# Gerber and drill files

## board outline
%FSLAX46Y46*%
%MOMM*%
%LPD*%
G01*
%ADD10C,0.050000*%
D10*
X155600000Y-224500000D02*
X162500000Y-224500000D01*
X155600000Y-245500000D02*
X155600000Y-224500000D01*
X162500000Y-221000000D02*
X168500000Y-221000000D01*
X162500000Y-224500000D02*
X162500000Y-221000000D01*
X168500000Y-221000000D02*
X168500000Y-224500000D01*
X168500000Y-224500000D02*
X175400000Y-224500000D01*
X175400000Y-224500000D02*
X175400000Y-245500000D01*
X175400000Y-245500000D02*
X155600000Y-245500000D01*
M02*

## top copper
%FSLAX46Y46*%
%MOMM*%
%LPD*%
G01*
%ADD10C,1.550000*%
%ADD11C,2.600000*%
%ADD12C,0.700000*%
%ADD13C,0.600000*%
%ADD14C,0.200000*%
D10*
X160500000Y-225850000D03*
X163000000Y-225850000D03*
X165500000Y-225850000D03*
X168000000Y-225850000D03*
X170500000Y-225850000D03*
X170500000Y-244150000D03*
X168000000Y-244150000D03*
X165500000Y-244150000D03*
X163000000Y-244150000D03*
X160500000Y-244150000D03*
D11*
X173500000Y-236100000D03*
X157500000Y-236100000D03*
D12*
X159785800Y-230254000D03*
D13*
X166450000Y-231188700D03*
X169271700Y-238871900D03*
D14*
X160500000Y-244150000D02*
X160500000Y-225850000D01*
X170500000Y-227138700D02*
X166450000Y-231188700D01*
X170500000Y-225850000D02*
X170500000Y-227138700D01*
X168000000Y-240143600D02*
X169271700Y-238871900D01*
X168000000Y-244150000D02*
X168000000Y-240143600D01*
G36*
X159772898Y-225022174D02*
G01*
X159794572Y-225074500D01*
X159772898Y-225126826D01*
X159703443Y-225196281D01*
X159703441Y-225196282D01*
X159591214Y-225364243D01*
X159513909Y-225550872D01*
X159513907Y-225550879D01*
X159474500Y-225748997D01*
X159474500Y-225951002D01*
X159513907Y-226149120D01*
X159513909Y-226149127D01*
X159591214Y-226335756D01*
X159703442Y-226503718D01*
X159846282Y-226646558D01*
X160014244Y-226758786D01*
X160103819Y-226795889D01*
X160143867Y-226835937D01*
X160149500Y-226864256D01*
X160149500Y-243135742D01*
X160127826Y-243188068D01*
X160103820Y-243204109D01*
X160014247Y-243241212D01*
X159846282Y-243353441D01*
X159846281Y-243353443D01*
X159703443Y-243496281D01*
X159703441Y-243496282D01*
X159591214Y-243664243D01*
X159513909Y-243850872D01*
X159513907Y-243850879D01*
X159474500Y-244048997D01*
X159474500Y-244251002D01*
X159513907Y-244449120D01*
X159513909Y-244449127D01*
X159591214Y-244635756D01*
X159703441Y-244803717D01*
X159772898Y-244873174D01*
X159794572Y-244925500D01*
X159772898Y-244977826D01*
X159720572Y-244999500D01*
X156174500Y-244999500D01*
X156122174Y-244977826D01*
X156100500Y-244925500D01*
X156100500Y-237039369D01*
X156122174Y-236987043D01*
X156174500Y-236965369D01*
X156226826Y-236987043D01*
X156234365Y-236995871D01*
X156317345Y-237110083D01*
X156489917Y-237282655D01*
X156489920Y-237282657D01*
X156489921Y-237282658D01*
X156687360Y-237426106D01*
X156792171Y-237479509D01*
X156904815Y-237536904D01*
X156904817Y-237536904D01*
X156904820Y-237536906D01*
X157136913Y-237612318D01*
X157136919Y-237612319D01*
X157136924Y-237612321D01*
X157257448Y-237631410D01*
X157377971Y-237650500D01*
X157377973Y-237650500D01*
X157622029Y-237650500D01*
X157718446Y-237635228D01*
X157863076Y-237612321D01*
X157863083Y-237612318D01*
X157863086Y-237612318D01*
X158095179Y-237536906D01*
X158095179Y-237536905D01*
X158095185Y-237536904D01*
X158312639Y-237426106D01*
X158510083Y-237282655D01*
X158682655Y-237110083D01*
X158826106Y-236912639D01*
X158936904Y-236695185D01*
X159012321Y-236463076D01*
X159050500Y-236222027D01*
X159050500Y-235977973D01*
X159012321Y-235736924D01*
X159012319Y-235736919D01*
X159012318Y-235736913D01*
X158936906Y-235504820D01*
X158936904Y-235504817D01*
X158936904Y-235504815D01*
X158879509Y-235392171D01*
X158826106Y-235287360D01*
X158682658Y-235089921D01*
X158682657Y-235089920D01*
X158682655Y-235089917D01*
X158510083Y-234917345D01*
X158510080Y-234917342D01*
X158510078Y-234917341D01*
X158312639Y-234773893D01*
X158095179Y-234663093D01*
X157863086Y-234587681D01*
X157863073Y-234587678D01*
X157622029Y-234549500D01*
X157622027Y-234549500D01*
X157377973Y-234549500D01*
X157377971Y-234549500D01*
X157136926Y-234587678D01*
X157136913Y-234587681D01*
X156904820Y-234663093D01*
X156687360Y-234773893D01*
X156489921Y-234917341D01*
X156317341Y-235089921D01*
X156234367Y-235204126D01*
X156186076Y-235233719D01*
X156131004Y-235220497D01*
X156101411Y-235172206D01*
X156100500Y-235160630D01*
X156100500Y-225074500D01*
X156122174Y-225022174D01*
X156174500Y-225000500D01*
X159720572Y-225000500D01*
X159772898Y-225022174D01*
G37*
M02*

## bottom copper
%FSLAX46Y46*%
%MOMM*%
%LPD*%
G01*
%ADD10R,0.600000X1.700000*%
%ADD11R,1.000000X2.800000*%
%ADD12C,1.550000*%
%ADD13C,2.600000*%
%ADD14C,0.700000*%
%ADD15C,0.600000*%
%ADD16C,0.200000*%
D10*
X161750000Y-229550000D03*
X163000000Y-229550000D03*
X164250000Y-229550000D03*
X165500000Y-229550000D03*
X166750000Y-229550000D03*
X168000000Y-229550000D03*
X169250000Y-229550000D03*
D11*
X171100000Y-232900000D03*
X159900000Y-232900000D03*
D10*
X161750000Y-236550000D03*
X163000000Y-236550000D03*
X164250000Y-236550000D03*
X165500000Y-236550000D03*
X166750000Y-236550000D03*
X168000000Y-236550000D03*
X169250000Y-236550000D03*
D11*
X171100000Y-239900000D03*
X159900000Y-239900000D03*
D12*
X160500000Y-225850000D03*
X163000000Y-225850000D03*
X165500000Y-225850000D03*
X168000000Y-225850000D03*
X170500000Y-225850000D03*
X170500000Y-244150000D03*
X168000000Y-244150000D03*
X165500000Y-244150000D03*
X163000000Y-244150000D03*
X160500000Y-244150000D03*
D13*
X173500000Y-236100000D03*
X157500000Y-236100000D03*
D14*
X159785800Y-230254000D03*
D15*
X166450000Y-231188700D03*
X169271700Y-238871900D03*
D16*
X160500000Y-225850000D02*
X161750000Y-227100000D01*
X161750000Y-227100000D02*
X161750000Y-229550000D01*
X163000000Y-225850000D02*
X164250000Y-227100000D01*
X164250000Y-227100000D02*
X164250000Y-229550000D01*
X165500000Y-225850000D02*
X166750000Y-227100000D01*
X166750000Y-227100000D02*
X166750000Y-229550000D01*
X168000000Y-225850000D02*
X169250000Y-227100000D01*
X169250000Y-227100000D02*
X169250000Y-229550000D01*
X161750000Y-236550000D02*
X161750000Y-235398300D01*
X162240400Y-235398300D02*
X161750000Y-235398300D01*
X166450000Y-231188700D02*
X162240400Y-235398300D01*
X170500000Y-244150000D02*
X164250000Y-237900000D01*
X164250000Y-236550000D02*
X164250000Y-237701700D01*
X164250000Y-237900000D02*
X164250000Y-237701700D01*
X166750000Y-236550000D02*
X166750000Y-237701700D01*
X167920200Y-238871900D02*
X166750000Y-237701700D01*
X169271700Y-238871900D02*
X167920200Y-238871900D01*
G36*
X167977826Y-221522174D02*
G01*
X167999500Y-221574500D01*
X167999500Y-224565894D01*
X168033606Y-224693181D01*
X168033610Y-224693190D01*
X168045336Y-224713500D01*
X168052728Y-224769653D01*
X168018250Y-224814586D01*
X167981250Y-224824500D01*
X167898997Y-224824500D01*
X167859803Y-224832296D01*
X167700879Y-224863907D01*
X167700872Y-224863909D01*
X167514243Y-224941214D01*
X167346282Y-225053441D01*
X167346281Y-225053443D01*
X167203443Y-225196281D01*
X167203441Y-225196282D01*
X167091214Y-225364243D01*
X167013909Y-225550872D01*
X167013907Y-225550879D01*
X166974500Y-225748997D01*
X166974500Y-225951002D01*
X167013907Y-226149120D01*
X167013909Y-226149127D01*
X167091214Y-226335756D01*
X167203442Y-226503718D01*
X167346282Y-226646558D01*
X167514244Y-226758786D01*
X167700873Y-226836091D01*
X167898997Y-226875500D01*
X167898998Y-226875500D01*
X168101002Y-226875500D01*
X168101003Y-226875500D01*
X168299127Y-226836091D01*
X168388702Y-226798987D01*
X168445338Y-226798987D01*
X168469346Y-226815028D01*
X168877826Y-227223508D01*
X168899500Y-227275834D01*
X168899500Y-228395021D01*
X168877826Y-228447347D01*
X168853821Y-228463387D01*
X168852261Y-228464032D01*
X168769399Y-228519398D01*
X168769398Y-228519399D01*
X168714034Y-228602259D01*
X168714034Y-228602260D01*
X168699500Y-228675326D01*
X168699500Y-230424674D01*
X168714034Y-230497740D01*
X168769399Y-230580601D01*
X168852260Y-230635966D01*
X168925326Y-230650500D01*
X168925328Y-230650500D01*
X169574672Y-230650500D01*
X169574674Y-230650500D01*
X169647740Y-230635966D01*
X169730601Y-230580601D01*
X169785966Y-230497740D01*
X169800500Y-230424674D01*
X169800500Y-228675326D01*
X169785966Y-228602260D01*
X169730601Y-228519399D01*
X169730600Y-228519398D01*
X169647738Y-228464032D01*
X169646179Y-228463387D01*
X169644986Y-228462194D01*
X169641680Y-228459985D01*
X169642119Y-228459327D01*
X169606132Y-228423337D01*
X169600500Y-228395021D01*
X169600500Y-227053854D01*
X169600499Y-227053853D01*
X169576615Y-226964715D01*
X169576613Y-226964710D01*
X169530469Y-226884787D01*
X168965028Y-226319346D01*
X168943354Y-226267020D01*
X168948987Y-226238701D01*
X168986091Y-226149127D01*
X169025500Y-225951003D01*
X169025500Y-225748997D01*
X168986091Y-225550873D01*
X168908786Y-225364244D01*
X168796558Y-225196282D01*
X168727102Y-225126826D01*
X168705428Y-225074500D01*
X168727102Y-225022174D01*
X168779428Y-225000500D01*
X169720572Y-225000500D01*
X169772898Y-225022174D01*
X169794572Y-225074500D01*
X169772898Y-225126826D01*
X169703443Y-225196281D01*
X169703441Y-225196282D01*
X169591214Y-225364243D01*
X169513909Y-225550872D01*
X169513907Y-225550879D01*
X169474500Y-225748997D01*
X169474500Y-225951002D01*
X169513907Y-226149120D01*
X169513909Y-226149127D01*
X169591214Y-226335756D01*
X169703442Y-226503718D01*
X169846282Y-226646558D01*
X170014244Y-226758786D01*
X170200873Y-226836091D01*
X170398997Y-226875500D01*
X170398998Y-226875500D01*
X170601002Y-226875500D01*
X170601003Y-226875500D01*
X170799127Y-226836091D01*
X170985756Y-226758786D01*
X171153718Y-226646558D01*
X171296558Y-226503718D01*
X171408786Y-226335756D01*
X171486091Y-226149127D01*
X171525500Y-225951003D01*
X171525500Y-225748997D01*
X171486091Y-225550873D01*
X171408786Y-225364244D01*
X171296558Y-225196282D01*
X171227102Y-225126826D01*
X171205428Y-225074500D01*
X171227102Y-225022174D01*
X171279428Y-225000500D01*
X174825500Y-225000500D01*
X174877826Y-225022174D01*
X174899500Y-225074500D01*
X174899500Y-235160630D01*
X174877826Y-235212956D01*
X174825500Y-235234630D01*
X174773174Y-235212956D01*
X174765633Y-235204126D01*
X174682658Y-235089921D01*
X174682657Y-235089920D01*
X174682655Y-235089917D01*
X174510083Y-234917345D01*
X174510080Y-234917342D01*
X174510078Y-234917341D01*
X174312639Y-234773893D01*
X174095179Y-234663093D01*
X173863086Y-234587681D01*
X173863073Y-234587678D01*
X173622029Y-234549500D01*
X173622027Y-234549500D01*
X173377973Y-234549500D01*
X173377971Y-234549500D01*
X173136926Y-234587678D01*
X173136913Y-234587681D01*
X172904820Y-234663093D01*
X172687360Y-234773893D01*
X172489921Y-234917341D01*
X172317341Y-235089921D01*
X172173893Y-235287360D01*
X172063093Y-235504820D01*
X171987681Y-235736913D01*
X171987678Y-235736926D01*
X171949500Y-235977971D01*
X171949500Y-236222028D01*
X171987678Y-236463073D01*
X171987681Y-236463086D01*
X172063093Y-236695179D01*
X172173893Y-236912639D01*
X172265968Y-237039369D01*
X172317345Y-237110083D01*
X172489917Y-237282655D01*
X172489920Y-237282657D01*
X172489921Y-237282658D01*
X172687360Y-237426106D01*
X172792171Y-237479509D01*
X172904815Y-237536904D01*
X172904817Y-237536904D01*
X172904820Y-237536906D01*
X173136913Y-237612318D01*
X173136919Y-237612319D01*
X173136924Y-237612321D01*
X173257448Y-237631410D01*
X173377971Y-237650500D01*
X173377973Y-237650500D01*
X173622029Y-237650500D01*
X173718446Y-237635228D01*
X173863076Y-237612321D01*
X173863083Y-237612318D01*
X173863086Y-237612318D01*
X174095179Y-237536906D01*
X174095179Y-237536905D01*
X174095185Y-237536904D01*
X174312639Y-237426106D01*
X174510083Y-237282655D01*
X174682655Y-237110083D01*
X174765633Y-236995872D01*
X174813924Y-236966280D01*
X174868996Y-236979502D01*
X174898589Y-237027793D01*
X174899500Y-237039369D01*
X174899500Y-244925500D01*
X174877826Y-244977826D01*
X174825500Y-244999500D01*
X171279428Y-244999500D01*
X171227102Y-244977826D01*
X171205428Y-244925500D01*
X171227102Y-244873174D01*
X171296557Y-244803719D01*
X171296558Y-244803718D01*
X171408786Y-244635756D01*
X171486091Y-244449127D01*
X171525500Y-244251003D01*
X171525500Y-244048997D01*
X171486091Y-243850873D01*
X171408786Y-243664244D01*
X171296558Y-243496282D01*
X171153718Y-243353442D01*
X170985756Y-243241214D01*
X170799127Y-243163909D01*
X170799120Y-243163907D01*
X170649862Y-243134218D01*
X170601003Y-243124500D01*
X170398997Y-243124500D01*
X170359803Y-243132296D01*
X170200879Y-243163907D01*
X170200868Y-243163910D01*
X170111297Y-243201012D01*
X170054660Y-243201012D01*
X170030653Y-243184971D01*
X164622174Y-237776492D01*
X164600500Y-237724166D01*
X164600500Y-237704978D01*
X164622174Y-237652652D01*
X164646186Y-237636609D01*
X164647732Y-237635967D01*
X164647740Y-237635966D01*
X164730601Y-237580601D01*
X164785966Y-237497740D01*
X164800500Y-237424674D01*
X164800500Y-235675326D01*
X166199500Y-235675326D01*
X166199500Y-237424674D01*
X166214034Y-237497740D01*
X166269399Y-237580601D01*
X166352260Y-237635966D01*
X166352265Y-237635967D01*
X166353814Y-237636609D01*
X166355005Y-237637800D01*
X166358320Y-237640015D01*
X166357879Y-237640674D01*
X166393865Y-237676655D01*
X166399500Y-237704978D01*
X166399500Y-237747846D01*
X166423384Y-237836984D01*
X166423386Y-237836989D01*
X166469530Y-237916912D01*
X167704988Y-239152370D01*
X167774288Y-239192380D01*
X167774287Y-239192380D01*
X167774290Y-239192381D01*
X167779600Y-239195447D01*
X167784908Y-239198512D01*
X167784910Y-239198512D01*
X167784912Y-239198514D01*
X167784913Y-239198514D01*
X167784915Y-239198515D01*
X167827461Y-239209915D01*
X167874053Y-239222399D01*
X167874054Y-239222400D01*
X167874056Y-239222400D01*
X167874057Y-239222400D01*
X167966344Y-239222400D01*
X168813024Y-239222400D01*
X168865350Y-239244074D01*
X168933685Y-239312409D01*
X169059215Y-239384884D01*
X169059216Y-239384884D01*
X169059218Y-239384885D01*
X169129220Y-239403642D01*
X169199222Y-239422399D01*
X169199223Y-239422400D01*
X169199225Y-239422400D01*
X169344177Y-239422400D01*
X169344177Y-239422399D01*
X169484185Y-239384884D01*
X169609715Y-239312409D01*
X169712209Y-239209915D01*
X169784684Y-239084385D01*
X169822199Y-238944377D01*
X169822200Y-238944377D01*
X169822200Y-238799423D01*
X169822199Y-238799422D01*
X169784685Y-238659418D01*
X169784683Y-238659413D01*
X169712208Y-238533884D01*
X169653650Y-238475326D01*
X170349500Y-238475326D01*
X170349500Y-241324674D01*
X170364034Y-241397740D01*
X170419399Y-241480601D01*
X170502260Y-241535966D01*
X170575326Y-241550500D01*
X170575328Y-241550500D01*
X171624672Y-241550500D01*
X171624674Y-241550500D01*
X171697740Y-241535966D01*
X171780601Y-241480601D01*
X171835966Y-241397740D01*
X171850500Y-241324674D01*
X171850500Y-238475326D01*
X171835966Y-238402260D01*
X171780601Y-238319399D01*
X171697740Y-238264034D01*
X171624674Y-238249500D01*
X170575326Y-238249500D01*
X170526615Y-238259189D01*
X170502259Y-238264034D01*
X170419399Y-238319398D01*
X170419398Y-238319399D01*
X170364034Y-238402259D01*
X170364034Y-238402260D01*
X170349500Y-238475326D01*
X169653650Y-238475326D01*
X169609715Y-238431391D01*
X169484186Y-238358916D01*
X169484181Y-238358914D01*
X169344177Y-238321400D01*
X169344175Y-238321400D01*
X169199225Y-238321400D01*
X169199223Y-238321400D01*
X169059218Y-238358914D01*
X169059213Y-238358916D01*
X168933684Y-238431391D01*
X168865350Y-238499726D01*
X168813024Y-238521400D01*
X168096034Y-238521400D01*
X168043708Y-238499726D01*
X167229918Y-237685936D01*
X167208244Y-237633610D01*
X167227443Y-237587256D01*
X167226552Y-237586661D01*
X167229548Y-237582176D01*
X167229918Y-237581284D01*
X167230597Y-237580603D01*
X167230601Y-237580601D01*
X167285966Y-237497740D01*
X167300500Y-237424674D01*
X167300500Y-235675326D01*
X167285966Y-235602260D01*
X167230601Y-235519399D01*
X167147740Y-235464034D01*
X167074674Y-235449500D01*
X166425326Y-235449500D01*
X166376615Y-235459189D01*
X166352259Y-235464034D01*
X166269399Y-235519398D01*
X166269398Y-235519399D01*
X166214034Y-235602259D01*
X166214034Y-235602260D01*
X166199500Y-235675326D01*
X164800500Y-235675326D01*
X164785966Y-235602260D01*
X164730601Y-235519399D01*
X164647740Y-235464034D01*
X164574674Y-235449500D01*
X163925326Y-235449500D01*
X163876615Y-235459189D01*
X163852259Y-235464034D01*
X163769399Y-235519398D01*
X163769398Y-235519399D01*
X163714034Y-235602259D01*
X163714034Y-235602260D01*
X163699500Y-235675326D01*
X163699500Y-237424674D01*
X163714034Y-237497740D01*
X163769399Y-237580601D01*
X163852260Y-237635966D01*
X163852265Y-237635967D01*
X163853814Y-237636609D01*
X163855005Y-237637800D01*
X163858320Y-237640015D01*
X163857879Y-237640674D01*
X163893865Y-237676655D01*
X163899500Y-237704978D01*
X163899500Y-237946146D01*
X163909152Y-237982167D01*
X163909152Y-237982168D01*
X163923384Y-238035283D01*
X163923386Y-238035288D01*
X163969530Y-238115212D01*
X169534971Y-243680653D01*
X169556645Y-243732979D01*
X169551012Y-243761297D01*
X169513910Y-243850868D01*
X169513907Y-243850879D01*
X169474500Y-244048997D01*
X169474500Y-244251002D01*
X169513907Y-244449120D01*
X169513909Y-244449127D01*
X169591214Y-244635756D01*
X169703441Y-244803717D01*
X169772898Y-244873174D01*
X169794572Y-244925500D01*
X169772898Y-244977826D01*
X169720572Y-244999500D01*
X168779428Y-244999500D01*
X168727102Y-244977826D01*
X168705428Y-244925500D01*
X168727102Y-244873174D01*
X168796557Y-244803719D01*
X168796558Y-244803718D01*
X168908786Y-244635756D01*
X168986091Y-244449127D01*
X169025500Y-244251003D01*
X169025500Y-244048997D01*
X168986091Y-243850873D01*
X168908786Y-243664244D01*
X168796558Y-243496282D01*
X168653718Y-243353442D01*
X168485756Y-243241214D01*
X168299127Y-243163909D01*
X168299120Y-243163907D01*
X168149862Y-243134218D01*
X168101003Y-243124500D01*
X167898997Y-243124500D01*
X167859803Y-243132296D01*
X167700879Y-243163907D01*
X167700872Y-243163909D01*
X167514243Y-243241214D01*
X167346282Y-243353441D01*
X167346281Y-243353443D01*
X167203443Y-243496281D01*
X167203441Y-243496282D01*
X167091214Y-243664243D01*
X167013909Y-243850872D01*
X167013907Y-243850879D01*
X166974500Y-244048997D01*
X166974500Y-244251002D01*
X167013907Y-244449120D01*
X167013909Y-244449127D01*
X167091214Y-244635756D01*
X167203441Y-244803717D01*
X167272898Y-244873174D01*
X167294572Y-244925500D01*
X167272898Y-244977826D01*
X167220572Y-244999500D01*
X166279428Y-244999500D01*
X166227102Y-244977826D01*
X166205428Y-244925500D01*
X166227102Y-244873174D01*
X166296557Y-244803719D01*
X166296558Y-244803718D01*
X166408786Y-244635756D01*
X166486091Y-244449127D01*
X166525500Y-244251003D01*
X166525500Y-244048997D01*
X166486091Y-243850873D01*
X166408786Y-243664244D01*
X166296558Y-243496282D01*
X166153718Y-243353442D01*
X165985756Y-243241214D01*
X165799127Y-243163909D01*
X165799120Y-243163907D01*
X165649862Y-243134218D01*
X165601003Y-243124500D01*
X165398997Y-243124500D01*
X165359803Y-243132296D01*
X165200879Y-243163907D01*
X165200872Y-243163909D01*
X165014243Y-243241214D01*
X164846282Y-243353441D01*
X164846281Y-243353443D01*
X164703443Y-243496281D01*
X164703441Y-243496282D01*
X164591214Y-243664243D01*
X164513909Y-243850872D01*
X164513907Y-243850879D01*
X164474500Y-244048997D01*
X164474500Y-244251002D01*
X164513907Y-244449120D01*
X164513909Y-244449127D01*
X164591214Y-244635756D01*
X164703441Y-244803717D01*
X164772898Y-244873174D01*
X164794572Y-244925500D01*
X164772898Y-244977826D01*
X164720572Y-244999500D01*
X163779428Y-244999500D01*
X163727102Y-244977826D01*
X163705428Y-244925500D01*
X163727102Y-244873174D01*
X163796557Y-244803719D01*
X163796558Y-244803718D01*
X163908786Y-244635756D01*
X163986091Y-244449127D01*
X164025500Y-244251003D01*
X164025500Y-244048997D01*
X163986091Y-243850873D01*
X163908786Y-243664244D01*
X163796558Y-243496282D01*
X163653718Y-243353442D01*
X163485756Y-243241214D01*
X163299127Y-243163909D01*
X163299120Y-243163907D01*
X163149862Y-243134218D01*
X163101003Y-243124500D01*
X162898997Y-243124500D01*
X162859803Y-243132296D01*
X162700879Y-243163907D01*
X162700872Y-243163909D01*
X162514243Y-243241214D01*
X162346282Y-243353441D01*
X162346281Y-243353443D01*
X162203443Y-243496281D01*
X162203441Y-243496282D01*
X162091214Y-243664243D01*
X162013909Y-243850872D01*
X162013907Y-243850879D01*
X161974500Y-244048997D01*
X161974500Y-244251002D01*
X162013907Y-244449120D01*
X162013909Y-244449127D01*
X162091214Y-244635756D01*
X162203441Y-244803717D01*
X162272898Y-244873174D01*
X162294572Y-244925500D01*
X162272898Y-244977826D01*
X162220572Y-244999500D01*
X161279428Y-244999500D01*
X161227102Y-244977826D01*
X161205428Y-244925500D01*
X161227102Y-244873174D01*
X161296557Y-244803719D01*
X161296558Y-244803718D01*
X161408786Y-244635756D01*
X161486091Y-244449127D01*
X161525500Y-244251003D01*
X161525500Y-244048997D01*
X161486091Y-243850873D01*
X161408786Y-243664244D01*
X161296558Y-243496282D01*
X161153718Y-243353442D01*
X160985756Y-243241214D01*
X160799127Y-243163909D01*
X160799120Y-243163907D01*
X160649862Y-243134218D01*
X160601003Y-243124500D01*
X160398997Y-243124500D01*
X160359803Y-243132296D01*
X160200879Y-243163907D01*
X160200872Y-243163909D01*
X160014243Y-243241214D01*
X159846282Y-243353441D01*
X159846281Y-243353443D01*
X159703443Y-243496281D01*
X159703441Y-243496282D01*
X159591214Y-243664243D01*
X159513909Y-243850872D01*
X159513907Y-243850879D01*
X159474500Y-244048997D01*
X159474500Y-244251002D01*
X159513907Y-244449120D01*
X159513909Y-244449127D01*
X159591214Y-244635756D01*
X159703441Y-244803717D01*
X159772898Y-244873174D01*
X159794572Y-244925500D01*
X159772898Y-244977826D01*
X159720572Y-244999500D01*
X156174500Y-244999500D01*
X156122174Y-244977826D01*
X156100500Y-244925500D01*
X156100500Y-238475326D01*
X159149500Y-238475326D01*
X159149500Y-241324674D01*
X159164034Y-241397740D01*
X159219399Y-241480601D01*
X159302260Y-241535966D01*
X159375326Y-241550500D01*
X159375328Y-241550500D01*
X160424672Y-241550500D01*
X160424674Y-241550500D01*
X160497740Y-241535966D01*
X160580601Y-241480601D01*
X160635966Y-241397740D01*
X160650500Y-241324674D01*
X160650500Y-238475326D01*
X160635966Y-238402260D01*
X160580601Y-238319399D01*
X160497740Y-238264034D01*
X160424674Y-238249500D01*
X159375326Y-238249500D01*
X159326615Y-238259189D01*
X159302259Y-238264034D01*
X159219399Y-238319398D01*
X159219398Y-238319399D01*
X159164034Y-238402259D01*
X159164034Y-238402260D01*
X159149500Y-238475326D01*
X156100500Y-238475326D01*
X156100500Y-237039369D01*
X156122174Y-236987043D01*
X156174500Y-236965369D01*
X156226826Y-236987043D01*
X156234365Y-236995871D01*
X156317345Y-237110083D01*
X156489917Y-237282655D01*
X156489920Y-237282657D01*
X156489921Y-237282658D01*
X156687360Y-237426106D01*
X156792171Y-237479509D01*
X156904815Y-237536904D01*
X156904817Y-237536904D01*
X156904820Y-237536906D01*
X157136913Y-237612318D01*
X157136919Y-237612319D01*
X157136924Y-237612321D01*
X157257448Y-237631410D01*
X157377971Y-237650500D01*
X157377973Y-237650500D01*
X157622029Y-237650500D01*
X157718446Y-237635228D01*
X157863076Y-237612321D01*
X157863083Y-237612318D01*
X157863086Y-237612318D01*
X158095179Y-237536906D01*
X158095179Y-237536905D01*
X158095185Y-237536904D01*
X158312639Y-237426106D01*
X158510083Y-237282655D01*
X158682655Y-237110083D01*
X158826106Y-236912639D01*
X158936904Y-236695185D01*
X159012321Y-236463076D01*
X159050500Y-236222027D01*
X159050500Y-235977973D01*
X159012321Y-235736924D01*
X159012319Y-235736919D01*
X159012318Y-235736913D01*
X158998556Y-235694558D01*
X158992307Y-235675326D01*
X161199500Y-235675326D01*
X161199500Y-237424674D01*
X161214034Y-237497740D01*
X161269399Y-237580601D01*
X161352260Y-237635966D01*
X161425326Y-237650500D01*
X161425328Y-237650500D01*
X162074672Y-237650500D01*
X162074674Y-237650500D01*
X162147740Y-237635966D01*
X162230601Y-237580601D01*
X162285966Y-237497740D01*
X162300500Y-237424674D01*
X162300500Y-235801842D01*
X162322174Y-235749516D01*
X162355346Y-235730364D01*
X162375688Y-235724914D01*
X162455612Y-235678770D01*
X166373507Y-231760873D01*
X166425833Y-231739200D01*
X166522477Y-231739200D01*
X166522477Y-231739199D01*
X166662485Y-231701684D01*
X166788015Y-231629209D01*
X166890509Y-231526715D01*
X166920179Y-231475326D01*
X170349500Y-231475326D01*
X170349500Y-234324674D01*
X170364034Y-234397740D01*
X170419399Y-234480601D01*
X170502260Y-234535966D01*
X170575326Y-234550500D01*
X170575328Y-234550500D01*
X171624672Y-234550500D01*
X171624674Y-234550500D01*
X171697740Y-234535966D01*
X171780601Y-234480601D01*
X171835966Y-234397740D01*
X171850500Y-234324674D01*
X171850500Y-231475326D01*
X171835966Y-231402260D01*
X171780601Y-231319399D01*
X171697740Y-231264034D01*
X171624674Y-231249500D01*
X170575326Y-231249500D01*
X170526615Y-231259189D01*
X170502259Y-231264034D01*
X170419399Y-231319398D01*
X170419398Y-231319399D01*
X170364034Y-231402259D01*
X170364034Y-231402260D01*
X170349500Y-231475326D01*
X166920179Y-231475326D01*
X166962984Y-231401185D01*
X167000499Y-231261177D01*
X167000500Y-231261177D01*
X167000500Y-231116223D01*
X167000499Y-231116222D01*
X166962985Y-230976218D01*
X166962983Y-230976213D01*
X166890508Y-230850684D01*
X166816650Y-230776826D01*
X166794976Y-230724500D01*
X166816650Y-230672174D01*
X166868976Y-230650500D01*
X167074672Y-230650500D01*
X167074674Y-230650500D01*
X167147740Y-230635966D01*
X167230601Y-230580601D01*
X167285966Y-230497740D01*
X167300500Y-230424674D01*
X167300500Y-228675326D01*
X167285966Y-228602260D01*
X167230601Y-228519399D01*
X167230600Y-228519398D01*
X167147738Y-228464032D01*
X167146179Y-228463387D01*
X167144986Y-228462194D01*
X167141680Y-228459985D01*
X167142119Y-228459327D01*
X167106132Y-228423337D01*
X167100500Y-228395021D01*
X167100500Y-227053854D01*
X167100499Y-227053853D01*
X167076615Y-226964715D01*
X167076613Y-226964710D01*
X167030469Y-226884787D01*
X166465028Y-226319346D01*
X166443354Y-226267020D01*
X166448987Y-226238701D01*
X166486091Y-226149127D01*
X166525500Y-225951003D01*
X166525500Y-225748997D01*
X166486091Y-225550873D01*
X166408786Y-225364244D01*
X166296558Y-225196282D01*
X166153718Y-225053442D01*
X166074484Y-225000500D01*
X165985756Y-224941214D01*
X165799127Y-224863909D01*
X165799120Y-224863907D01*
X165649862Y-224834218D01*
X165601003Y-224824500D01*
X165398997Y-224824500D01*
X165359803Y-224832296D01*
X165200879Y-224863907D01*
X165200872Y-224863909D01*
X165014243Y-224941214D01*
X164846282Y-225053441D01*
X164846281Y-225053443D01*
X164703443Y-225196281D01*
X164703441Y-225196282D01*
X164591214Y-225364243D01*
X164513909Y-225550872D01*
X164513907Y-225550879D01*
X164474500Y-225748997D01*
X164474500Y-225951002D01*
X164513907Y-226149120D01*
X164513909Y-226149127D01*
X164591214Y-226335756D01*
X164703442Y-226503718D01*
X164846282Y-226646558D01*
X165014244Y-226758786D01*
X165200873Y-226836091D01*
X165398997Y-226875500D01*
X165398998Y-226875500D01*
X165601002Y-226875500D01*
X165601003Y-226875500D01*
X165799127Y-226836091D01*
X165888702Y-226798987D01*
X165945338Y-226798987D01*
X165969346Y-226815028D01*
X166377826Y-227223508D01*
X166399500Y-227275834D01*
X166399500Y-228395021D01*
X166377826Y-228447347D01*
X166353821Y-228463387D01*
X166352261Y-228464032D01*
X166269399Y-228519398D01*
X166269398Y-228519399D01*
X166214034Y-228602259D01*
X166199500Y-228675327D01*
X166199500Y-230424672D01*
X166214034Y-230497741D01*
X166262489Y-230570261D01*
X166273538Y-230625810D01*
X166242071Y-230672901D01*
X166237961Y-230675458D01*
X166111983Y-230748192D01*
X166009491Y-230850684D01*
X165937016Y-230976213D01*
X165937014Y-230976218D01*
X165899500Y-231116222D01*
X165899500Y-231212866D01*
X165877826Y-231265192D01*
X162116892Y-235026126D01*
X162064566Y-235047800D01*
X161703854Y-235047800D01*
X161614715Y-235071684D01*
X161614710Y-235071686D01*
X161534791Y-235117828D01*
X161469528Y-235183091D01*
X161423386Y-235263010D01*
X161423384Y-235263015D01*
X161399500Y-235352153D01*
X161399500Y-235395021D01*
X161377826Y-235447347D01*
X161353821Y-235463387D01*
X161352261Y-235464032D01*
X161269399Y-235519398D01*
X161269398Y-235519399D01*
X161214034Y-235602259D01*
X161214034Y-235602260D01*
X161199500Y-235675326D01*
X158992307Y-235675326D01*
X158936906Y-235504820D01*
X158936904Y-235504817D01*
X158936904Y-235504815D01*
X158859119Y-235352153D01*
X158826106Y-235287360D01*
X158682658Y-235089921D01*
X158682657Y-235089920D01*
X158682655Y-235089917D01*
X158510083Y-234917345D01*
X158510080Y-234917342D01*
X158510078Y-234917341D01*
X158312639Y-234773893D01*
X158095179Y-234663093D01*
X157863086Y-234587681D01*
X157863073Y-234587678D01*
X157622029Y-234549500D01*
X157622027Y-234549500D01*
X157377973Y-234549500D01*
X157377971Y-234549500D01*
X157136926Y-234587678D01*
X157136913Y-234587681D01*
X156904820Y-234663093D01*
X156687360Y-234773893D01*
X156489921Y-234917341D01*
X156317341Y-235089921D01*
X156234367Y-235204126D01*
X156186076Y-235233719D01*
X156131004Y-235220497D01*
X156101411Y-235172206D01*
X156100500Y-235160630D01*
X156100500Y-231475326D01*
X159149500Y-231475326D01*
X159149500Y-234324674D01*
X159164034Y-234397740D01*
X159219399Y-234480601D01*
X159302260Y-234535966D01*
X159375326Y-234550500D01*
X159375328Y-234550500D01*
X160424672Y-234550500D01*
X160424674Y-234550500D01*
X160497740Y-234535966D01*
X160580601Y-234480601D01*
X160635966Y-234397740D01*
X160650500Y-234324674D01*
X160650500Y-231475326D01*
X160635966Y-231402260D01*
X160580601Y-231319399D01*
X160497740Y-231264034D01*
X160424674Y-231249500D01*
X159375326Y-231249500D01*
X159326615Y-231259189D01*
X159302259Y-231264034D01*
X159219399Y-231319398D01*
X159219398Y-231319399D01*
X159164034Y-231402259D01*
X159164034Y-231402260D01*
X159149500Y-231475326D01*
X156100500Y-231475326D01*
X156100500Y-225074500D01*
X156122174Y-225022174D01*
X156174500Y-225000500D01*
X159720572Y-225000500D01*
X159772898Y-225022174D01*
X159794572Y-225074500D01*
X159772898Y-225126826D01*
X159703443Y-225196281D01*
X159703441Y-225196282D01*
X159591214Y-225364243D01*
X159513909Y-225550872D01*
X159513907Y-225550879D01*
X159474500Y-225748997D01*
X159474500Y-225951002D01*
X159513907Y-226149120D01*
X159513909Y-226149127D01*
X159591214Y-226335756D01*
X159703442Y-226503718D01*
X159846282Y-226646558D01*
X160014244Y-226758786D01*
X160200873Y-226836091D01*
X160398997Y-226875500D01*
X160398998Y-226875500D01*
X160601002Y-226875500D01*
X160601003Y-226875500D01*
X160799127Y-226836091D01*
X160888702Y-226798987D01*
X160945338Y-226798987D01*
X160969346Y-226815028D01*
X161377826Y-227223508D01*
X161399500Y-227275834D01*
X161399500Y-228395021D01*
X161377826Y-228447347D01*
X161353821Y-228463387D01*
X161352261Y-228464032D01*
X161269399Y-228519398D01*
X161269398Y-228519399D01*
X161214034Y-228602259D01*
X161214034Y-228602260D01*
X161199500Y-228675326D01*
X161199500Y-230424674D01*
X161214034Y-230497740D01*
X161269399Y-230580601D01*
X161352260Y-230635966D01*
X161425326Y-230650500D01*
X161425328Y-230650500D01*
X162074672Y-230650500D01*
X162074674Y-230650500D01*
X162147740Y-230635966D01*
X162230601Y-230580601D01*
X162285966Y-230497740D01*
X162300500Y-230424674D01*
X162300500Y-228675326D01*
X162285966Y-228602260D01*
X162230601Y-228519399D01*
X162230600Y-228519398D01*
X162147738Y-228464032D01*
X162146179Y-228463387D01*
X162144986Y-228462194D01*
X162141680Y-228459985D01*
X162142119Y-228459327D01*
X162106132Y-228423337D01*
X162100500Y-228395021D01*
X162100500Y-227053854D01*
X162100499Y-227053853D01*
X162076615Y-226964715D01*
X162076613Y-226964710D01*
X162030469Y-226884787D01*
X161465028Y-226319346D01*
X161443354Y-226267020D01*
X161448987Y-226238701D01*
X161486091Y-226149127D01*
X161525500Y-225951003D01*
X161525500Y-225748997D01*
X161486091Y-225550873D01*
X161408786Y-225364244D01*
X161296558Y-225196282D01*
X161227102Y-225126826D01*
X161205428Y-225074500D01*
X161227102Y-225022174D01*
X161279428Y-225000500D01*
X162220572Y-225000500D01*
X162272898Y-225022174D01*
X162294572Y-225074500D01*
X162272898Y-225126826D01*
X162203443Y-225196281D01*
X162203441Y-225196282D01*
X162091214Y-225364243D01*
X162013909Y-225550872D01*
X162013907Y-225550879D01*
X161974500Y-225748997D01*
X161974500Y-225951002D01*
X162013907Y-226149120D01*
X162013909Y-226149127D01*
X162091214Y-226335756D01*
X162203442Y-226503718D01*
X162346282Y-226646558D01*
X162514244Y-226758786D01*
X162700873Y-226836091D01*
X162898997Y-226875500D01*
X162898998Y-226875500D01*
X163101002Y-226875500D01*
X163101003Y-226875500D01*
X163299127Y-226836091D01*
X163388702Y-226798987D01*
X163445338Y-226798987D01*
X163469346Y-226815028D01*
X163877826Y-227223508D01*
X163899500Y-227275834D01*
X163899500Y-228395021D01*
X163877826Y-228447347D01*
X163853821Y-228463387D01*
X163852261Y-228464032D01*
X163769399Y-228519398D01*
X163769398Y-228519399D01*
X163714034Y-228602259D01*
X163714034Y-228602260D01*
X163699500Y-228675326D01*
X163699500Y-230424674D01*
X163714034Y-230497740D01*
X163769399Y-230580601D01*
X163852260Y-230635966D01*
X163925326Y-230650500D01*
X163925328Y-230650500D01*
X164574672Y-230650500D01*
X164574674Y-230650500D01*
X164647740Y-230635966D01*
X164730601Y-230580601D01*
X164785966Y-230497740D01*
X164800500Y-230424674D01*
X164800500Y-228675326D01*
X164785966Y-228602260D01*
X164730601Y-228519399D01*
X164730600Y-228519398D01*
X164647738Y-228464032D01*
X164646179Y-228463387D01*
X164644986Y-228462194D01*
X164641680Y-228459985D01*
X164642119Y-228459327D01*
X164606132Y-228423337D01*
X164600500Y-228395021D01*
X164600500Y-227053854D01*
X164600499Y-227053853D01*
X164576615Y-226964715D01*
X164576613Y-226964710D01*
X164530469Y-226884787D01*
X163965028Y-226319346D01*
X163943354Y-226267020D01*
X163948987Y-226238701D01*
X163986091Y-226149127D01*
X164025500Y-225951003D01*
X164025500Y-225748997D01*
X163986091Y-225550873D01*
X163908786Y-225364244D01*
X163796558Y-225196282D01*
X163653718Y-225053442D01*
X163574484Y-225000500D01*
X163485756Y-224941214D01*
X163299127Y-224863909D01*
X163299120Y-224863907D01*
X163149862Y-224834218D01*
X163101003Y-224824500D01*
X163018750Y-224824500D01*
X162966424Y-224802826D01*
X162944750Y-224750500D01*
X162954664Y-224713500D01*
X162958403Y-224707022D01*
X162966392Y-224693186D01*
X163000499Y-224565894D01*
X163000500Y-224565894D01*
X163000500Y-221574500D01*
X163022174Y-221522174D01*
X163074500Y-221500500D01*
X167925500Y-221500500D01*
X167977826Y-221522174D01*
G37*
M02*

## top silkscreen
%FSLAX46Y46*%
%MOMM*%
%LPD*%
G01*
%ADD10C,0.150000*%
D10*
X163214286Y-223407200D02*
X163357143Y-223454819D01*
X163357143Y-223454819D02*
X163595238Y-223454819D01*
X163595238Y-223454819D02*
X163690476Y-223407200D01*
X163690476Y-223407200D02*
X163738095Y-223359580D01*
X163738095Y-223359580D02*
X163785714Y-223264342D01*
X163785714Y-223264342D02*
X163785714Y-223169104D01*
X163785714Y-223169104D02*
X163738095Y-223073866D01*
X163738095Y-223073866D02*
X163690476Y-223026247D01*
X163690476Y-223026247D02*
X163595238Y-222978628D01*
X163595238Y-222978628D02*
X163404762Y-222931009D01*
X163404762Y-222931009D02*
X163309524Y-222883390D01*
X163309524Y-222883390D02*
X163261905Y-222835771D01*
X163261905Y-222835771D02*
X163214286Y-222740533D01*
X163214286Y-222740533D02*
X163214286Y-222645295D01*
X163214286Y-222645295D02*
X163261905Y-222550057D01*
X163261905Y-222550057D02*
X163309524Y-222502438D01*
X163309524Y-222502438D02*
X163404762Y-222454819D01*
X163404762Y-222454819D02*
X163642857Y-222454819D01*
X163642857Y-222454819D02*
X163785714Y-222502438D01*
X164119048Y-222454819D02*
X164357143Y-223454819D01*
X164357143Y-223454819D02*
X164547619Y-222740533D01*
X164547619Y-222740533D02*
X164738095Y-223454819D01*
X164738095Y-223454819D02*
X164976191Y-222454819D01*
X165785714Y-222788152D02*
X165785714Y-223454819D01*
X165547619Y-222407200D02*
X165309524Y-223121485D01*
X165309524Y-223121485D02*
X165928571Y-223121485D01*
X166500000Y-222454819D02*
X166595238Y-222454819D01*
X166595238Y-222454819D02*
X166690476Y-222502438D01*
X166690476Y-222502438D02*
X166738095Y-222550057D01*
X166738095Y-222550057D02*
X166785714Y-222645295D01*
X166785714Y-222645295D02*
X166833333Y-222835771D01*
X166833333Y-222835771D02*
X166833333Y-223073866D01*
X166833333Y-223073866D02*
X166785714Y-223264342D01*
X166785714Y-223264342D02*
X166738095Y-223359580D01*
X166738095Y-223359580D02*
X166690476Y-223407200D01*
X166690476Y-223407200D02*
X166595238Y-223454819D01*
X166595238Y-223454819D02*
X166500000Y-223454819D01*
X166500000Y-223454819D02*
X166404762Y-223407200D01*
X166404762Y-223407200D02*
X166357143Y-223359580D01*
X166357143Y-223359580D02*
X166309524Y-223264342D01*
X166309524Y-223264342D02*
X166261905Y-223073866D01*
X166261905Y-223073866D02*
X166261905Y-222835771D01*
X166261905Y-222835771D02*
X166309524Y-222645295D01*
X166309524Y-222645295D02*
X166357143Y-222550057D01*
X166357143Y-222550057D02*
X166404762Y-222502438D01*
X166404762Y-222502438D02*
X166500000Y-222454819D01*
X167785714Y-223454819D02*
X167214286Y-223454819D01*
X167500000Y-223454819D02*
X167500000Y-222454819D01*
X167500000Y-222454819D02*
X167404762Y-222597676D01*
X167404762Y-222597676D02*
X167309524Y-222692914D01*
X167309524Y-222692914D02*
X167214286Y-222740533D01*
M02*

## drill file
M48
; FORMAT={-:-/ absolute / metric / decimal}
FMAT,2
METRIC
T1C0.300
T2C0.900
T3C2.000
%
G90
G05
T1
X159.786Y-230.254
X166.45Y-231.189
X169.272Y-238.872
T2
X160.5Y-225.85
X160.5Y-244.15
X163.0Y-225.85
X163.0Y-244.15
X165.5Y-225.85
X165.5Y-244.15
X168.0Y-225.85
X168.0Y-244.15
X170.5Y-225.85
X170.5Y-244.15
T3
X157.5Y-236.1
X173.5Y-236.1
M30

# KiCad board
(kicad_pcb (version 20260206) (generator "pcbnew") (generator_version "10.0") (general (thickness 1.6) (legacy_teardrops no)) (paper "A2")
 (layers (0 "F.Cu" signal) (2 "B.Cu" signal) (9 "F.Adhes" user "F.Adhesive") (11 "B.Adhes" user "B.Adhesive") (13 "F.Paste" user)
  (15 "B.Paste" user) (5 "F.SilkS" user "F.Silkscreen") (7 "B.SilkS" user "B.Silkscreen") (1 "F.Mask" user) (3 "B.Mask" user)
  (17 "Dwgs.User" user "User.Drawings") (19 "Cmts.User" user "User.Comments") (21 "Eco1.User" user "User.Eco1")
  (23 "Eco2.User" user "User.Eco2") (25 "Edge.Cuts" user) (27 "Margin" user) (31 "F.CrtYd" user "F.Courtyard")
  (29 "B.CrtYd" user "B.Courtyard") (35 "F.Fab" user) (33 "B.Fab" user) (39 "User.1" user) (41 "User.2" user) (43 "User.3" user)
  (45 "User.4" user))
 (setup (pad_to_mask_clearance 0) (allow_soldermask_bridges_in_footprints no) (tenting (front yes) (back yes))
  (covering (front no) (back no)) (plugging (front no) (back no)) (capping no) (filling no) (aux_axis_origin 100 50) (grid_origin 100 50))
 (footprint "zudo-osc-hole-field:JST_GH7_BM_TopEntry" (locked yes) (layer "B.Cu") (at 165.5 229.55 180)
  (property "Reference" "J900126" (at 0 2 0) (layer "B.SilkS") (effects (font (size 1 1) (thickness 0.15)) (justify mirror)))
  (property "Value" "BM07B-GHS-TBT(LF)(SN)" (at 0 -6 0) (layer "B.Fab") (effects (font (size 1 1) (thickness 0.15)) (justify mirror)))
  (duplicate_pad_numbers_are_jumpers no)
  (pad "1" smd rect (at 3.75 0 180) (size 0.6 1.7) (layers "B.Cu" "B.Mask" "B.Paste") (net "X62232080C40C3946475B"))
  (pad "2" smd rect (at 2.5 0 180) (size 0.6 1.7) (layers "B.Cu" "B.Mask" "B.Paste") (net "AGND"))
  (pad "3" smd rect (at 1.25 0 180) (size 0.6 1.7) (layers "B.Cu" "B.Mask" "B.Paste") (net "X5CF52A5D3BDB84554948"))
  (pad "4" smd rect (at 0 0 180) (size 0.6 1.7) (layers "B.Cu" "B.Mask" "B.Paste") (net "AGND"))
  (pad "5" smd rect (at -1.25 0 180) (size 0.6 1.7) (layers "B.Cu" "B.Mask" "B.Paste") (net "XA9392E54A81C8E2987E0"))
  (pad "6" smd rect (at -2.5 0 180) (size 0.6 1.7) (layers "B.Cu" "B.Mask" "B.Paste") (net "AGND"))
  (pad "7" smd rect (at -3.75 0 180) (size 0.6 1.7) (layers "B.Cu" "B.Mask" "B.Paste") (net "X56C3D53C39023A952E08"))
  (pad "MP1" smd rect (at -5.6 -3.35 180) (size 1 2.8) (layers "B.Cu" "B.Mask" "B.Paste") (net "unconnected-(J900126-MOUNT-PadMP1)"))
  (pad "MP2" smd rect (at 5.6 -3.35 180) (size 1 2.8) (layers "B.Cu" "B.Mask" "B.Paste") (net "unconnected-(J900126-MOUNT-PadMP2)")))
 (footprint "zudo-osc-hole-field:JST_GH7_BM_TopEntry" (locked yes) (layer "B.Cu") (at 165.5 236.55 180)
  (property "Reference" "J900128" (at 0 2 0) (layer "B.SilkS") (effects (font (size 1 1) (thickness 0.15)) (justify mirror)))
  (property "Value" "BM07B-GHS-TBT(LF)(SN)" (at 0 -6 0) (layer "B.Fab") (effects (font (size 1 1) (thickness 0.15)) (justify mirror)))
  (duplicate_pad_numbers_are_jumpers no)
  (pad "1" smd rect (at 3.75 0 180) (size 0.6 1.7) (layers "B.Cu" "B.Mask" "B.Paste") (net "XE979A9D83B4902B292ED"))
  (pad "2" smd rect (at 2.5 0 180) (size 0.6 1.7) (layers "B.Cu" "B.Mask" "B.Paste") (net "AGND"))
  (pad "3" smd rect (at 1.25 0 180) (size 0.6 1.7) (layers "B.Cu" "B.Mask" "B.Paste") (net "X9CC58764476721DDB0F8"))
  (pad "4" smd rect (at 0 0 180) (size 0.6 1.7) (layers "B.Cu" "B.Mask" "B.Paste") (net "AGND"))
  (pad "5" smd rect (at -1.25 0 180) (size 0.6 1.7) (layers "B.Cu" "B.Mask" "B.Paste") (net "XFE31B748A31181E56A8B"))
  (pad "6" smd rect (at -2.5 0 180) (size 0.6 1.7) (layers "B.Cu" "B.Mask" "B.Paste") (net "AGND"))
  (pad "7" smd rect (at -3.75 0 180) (size 0.6 1.7) (layers "B.Cu" "B.Mask" "B.Paste") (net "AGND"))
  (pad "MP1" smd rect (at -5.6 -3.35 180) (size 1 2.8) (layers "B.Cu" "B.Mask" "B.Paste") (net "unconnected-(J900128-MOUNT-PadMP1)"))
  (pad "MP2" smd rect (at 5.6 -3.35 180) (size 1 2.8) (layers "B.Cu" "B.Mask" "B.Paste") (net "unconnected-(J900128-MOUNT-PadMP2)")))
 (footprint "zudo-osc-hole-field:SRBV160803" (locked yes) (layer "F.Cu") (at 165.5 235 180)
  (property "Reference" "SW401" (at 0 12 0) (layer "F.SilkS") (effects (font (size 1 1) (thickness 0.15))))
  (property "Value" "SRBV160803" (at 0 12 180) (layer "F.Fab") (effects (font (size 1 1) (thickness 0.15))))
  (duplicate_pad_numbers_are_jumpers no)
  (pad "1" thru_hole circle (at 5 9.15 180) (size 1.55 1.55) (drill 0.9) (layers "*.Cu" "*.Mask") (remove_unused_layers no)
   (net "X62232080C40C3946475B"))
  (pad "2" thru_hole circle (at 2.5 9.15 180) (size 1.55 1.55) (drill 0.9) (layers "*.Cu" "*.Mask") (remove_unused_layers no)
   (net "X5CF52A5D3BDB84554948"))
  (pad "3" thru_hole circle (at 0 9.15 180) (size 1.55 1.55) (drill 0.9) (layers "*.Cu" "*.Mask") (remove_unused_layers no)
   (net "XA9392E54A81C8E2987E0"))
  (pad "4" thru_hole circle (at -2.5 9.15 180) (size 1.55 1.55) (drill 0.9) (layers "*.Cu" "*.Mask") (remove_unused_layers no)
   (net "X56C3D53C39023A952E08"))
  (pad "5" thru_hole circle (at -5 9.15 180) (size 1.55 1.55) (drill 0.9) (layers "*.Cu" "*.Mask") (remove_unused_layers no)
   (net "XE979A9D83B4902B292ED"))
  (pad "6" thru_hole circle (at -5 -9.15 180) (size 1.55 1.55) (drill 0.9) (layers "*.Cu" "*.Mask") (remove_unused_layers no)
   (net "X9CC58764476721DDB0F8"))
  (pad "7" thru_hole circle (at -2.5 -9.15 180) (size 1.55 1.55) (drill 0.9) (layers "*.Cu" "*.Mask") (remove_unused_layers no)
   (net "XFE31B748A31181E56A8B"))
  (pad "8" thru_hole circle (at 0 -9.15 180) (size 1.55 1.55) (drill 0.9) (layers "*.Cu" "*.Mask") (remove_unused_layers no)
   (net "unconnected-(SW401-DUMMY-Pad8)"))
  (pad "9" thru_hole circle (at 2.5 -9.15 180) (size 1.55 1.55) (drill 0.9) (layers "*.Cu" "*.Mask") (remove_unused_layers no)
   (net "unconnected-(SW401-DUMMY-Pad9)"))
  (pad "10" thru_hole circle (at 5 -9.15 180) (size 1.55 1.55) (drill 0.9) (layers "*.Cu" "*.Mask") (remove_unused_layers no)
   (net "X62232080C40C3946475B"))
  (pad "MP1" thru_hole circle (at -8 -1.1 180) (size 2.6 2.6) (drill 2) (layers "*.Cu" "*.Mask") (remove_unused_layers no)
   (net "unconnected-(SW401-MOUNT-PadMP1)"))
  (pad "MP2" thru_hole circle (at 8 -1.1 180) (size 2.6 2.6) (drill 2) (layers "*.Cu" "*.Mask") (remove_unused_layers no)
   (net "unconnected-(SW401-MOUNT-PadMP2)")))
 (gr_line (start 155.6 224.5) (end 162.5 224.5) (stroke (width 0.05) (type default)) (layer "Edge.Cuts"))
 (gr_line (start 155.6 245.5) (end 155.6 224.5) (stroke (width 0.05) (type default)) (layer "Edge.Cuts"))
 (gr_line (start 162.5 221) (end 168.5 221) (stroke (width 0.05) (type default)) (layer "Edge.Cuts"))
 (gr_line (start 162.5 224.5) (end 162.5 221) (stroke (width 0.05) (type default)) (layer "Edge.Cuts"))
 (gr_line (start 168.5 221) (end 168.5 224.5) (stroke (width 0.05) (type default)) (layer "Edge.Cuts"))
 (gr_line (start 168.5 224.5) (end 175.4 224.5) (stroke (width 0.05) (type default)) (layer "Edge.Cuts"))
 (gr_line (start 175.4 224.5) (end 175.4 245.5) (stroke (width 0.05) (type default)) (layer "Edge.Cuts"))
 (gr_line (start 175.4 245.5) (end 155.6 245.5) (stroke (width 0.05) (type default)) (layer "Edge.Cuts"))
 (segment (start 160.5 244.15) (end 160.5 225.85) (width 0.2) (layer "F.Cu") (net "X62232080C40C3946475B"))
 (segment (start 160.5 225.85) (end 161.75 227.1) (width 0.2) (layer "B.Cu") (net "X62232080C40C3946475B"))
 (segment (start 161.75 227.1) (end 161.75 229.55) (width 0.2) (layer "B.Cu") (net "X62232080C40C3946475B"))
 (via (at 159.7858 230.254) (size 0.7) (drill 0.3) (layers "F.Cu" "B.Cu") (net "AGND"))
 (segment (start 163 225.85) (end 164.25 227.1) (width 0.2) (layer "B.Cu") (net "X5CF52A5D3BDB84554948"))
 (segment (start 164.25 227.1) (end 164.25 229.55) (width 0.2) (layer "B.Cu") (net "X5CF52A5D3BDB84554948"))
 (segment (start 165.5 225.85) (end 166.75 227.1) (width 0.2) (layer "B.Cu") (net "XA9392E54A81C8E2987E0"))
 (segment (start 166.75 227.1) (end 166.75 229.55) (width 0.2) (layer "B.Cu") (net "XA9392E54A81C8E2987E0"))
 (segment (start 168 225.85) (end 169.25 227.1) (width 0.2) (layer "B.Cu") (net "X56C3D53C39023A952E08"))
 (segment (start 169.25 227.1) (end 169.25 229.55) (width 0.2) (layer "B.Cu") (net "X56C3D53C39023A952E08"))
 (segment (start 170.5 227.1387) (end 166.45 231.1887) (width 0.2) (layer "F.Cu") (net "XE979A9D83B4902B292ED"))
 (segment (start 170.5 225.85) (end 170.5 227.1387) (width 0.2) (layer "F.Cu") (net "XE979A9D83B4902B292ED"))
 (via (at 166.45 231.1887) (size 0.6) (drill 0.3) (layers "F.Cu" "B.Cu") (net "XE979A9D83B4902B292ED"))
 (segment (start 161.75 236.55) (end 161.75 235.3983) (width 0.2) (layer "B.Cu") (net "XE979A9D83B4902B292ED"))
 (segment (start 162.2404 235.3983) (end 161.75 235.3983) (width 0.2) (layer "B.Cu") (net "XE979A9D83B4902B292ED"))
 (segment (start 166.45 231.1887) (end 162.2404 235.3983) (width 0.2) (layer "B.Cu") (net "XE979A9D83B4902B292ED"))
 (segment (start 170.5 244.15) (end 164.25 237.9) (width 0.2) (layer "B.Cu") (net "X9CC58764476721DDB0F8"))
 (segment (start 164.25 236.55) (end 164.25 237.7017) (width 0.2) (layer "B.Cu") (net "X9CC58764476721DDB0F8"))
 (segment (start 164.25 237.9) (end 164.25 237.7017) (width 0.2) (layer "B.Cu") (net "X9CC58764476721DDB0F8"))
 (segment (start 168 240.1436) (end 169.2717 238.8719) (width 0.2) (layer "F.Cu") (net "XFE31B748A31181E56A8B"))
 (segment (start 168 244.15) (end 168 240.1436) (width 0.2) (layer "F.Cu") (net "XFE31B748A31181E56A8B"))
 (via (at 169.2717 238.8719) (size 0.6) (drill 0.3) (layers "F.Cu" "B.Cu") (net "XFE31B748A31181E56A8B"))
 (segment (start 166.75 236.55) (end 166.75 237.7017) (width 0.2) (layer "B.Cu") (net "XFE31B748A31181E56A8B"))
 (segment (start 167.9202 238.8719) (end 166.75 237.7017) (width 0.2) (layer "B.Cu") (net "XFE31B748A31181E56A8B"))
 (segment (start 169.2717 238.8719) (end 167.9202 238.8719) (width 0.2) (layer "B.Cu") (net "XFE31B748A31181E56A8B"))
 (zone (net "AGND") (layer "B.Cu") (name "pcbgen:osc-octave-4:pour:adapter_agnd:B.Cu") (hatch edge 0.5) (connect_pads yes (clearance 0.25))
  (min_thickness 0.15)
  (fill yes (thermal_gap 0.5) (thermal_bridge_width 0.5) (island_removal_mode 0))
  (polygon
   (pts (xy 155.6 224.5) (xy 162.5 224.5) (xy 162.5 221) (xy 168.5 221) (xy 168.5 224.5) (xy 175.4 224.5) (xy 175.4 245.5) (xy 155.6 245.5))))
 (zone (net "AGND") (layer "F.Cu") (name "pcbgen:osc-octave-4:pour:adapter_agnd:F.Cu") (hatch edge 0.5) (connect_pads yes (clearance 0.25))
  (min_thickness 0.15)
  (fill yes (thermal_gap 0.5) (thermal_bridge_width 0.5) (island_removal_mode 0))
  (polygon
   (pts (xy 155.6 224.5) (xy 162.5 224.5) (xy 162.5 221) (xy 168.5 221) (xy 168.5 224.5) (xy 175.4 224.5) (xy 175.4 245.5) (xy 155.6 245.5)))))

